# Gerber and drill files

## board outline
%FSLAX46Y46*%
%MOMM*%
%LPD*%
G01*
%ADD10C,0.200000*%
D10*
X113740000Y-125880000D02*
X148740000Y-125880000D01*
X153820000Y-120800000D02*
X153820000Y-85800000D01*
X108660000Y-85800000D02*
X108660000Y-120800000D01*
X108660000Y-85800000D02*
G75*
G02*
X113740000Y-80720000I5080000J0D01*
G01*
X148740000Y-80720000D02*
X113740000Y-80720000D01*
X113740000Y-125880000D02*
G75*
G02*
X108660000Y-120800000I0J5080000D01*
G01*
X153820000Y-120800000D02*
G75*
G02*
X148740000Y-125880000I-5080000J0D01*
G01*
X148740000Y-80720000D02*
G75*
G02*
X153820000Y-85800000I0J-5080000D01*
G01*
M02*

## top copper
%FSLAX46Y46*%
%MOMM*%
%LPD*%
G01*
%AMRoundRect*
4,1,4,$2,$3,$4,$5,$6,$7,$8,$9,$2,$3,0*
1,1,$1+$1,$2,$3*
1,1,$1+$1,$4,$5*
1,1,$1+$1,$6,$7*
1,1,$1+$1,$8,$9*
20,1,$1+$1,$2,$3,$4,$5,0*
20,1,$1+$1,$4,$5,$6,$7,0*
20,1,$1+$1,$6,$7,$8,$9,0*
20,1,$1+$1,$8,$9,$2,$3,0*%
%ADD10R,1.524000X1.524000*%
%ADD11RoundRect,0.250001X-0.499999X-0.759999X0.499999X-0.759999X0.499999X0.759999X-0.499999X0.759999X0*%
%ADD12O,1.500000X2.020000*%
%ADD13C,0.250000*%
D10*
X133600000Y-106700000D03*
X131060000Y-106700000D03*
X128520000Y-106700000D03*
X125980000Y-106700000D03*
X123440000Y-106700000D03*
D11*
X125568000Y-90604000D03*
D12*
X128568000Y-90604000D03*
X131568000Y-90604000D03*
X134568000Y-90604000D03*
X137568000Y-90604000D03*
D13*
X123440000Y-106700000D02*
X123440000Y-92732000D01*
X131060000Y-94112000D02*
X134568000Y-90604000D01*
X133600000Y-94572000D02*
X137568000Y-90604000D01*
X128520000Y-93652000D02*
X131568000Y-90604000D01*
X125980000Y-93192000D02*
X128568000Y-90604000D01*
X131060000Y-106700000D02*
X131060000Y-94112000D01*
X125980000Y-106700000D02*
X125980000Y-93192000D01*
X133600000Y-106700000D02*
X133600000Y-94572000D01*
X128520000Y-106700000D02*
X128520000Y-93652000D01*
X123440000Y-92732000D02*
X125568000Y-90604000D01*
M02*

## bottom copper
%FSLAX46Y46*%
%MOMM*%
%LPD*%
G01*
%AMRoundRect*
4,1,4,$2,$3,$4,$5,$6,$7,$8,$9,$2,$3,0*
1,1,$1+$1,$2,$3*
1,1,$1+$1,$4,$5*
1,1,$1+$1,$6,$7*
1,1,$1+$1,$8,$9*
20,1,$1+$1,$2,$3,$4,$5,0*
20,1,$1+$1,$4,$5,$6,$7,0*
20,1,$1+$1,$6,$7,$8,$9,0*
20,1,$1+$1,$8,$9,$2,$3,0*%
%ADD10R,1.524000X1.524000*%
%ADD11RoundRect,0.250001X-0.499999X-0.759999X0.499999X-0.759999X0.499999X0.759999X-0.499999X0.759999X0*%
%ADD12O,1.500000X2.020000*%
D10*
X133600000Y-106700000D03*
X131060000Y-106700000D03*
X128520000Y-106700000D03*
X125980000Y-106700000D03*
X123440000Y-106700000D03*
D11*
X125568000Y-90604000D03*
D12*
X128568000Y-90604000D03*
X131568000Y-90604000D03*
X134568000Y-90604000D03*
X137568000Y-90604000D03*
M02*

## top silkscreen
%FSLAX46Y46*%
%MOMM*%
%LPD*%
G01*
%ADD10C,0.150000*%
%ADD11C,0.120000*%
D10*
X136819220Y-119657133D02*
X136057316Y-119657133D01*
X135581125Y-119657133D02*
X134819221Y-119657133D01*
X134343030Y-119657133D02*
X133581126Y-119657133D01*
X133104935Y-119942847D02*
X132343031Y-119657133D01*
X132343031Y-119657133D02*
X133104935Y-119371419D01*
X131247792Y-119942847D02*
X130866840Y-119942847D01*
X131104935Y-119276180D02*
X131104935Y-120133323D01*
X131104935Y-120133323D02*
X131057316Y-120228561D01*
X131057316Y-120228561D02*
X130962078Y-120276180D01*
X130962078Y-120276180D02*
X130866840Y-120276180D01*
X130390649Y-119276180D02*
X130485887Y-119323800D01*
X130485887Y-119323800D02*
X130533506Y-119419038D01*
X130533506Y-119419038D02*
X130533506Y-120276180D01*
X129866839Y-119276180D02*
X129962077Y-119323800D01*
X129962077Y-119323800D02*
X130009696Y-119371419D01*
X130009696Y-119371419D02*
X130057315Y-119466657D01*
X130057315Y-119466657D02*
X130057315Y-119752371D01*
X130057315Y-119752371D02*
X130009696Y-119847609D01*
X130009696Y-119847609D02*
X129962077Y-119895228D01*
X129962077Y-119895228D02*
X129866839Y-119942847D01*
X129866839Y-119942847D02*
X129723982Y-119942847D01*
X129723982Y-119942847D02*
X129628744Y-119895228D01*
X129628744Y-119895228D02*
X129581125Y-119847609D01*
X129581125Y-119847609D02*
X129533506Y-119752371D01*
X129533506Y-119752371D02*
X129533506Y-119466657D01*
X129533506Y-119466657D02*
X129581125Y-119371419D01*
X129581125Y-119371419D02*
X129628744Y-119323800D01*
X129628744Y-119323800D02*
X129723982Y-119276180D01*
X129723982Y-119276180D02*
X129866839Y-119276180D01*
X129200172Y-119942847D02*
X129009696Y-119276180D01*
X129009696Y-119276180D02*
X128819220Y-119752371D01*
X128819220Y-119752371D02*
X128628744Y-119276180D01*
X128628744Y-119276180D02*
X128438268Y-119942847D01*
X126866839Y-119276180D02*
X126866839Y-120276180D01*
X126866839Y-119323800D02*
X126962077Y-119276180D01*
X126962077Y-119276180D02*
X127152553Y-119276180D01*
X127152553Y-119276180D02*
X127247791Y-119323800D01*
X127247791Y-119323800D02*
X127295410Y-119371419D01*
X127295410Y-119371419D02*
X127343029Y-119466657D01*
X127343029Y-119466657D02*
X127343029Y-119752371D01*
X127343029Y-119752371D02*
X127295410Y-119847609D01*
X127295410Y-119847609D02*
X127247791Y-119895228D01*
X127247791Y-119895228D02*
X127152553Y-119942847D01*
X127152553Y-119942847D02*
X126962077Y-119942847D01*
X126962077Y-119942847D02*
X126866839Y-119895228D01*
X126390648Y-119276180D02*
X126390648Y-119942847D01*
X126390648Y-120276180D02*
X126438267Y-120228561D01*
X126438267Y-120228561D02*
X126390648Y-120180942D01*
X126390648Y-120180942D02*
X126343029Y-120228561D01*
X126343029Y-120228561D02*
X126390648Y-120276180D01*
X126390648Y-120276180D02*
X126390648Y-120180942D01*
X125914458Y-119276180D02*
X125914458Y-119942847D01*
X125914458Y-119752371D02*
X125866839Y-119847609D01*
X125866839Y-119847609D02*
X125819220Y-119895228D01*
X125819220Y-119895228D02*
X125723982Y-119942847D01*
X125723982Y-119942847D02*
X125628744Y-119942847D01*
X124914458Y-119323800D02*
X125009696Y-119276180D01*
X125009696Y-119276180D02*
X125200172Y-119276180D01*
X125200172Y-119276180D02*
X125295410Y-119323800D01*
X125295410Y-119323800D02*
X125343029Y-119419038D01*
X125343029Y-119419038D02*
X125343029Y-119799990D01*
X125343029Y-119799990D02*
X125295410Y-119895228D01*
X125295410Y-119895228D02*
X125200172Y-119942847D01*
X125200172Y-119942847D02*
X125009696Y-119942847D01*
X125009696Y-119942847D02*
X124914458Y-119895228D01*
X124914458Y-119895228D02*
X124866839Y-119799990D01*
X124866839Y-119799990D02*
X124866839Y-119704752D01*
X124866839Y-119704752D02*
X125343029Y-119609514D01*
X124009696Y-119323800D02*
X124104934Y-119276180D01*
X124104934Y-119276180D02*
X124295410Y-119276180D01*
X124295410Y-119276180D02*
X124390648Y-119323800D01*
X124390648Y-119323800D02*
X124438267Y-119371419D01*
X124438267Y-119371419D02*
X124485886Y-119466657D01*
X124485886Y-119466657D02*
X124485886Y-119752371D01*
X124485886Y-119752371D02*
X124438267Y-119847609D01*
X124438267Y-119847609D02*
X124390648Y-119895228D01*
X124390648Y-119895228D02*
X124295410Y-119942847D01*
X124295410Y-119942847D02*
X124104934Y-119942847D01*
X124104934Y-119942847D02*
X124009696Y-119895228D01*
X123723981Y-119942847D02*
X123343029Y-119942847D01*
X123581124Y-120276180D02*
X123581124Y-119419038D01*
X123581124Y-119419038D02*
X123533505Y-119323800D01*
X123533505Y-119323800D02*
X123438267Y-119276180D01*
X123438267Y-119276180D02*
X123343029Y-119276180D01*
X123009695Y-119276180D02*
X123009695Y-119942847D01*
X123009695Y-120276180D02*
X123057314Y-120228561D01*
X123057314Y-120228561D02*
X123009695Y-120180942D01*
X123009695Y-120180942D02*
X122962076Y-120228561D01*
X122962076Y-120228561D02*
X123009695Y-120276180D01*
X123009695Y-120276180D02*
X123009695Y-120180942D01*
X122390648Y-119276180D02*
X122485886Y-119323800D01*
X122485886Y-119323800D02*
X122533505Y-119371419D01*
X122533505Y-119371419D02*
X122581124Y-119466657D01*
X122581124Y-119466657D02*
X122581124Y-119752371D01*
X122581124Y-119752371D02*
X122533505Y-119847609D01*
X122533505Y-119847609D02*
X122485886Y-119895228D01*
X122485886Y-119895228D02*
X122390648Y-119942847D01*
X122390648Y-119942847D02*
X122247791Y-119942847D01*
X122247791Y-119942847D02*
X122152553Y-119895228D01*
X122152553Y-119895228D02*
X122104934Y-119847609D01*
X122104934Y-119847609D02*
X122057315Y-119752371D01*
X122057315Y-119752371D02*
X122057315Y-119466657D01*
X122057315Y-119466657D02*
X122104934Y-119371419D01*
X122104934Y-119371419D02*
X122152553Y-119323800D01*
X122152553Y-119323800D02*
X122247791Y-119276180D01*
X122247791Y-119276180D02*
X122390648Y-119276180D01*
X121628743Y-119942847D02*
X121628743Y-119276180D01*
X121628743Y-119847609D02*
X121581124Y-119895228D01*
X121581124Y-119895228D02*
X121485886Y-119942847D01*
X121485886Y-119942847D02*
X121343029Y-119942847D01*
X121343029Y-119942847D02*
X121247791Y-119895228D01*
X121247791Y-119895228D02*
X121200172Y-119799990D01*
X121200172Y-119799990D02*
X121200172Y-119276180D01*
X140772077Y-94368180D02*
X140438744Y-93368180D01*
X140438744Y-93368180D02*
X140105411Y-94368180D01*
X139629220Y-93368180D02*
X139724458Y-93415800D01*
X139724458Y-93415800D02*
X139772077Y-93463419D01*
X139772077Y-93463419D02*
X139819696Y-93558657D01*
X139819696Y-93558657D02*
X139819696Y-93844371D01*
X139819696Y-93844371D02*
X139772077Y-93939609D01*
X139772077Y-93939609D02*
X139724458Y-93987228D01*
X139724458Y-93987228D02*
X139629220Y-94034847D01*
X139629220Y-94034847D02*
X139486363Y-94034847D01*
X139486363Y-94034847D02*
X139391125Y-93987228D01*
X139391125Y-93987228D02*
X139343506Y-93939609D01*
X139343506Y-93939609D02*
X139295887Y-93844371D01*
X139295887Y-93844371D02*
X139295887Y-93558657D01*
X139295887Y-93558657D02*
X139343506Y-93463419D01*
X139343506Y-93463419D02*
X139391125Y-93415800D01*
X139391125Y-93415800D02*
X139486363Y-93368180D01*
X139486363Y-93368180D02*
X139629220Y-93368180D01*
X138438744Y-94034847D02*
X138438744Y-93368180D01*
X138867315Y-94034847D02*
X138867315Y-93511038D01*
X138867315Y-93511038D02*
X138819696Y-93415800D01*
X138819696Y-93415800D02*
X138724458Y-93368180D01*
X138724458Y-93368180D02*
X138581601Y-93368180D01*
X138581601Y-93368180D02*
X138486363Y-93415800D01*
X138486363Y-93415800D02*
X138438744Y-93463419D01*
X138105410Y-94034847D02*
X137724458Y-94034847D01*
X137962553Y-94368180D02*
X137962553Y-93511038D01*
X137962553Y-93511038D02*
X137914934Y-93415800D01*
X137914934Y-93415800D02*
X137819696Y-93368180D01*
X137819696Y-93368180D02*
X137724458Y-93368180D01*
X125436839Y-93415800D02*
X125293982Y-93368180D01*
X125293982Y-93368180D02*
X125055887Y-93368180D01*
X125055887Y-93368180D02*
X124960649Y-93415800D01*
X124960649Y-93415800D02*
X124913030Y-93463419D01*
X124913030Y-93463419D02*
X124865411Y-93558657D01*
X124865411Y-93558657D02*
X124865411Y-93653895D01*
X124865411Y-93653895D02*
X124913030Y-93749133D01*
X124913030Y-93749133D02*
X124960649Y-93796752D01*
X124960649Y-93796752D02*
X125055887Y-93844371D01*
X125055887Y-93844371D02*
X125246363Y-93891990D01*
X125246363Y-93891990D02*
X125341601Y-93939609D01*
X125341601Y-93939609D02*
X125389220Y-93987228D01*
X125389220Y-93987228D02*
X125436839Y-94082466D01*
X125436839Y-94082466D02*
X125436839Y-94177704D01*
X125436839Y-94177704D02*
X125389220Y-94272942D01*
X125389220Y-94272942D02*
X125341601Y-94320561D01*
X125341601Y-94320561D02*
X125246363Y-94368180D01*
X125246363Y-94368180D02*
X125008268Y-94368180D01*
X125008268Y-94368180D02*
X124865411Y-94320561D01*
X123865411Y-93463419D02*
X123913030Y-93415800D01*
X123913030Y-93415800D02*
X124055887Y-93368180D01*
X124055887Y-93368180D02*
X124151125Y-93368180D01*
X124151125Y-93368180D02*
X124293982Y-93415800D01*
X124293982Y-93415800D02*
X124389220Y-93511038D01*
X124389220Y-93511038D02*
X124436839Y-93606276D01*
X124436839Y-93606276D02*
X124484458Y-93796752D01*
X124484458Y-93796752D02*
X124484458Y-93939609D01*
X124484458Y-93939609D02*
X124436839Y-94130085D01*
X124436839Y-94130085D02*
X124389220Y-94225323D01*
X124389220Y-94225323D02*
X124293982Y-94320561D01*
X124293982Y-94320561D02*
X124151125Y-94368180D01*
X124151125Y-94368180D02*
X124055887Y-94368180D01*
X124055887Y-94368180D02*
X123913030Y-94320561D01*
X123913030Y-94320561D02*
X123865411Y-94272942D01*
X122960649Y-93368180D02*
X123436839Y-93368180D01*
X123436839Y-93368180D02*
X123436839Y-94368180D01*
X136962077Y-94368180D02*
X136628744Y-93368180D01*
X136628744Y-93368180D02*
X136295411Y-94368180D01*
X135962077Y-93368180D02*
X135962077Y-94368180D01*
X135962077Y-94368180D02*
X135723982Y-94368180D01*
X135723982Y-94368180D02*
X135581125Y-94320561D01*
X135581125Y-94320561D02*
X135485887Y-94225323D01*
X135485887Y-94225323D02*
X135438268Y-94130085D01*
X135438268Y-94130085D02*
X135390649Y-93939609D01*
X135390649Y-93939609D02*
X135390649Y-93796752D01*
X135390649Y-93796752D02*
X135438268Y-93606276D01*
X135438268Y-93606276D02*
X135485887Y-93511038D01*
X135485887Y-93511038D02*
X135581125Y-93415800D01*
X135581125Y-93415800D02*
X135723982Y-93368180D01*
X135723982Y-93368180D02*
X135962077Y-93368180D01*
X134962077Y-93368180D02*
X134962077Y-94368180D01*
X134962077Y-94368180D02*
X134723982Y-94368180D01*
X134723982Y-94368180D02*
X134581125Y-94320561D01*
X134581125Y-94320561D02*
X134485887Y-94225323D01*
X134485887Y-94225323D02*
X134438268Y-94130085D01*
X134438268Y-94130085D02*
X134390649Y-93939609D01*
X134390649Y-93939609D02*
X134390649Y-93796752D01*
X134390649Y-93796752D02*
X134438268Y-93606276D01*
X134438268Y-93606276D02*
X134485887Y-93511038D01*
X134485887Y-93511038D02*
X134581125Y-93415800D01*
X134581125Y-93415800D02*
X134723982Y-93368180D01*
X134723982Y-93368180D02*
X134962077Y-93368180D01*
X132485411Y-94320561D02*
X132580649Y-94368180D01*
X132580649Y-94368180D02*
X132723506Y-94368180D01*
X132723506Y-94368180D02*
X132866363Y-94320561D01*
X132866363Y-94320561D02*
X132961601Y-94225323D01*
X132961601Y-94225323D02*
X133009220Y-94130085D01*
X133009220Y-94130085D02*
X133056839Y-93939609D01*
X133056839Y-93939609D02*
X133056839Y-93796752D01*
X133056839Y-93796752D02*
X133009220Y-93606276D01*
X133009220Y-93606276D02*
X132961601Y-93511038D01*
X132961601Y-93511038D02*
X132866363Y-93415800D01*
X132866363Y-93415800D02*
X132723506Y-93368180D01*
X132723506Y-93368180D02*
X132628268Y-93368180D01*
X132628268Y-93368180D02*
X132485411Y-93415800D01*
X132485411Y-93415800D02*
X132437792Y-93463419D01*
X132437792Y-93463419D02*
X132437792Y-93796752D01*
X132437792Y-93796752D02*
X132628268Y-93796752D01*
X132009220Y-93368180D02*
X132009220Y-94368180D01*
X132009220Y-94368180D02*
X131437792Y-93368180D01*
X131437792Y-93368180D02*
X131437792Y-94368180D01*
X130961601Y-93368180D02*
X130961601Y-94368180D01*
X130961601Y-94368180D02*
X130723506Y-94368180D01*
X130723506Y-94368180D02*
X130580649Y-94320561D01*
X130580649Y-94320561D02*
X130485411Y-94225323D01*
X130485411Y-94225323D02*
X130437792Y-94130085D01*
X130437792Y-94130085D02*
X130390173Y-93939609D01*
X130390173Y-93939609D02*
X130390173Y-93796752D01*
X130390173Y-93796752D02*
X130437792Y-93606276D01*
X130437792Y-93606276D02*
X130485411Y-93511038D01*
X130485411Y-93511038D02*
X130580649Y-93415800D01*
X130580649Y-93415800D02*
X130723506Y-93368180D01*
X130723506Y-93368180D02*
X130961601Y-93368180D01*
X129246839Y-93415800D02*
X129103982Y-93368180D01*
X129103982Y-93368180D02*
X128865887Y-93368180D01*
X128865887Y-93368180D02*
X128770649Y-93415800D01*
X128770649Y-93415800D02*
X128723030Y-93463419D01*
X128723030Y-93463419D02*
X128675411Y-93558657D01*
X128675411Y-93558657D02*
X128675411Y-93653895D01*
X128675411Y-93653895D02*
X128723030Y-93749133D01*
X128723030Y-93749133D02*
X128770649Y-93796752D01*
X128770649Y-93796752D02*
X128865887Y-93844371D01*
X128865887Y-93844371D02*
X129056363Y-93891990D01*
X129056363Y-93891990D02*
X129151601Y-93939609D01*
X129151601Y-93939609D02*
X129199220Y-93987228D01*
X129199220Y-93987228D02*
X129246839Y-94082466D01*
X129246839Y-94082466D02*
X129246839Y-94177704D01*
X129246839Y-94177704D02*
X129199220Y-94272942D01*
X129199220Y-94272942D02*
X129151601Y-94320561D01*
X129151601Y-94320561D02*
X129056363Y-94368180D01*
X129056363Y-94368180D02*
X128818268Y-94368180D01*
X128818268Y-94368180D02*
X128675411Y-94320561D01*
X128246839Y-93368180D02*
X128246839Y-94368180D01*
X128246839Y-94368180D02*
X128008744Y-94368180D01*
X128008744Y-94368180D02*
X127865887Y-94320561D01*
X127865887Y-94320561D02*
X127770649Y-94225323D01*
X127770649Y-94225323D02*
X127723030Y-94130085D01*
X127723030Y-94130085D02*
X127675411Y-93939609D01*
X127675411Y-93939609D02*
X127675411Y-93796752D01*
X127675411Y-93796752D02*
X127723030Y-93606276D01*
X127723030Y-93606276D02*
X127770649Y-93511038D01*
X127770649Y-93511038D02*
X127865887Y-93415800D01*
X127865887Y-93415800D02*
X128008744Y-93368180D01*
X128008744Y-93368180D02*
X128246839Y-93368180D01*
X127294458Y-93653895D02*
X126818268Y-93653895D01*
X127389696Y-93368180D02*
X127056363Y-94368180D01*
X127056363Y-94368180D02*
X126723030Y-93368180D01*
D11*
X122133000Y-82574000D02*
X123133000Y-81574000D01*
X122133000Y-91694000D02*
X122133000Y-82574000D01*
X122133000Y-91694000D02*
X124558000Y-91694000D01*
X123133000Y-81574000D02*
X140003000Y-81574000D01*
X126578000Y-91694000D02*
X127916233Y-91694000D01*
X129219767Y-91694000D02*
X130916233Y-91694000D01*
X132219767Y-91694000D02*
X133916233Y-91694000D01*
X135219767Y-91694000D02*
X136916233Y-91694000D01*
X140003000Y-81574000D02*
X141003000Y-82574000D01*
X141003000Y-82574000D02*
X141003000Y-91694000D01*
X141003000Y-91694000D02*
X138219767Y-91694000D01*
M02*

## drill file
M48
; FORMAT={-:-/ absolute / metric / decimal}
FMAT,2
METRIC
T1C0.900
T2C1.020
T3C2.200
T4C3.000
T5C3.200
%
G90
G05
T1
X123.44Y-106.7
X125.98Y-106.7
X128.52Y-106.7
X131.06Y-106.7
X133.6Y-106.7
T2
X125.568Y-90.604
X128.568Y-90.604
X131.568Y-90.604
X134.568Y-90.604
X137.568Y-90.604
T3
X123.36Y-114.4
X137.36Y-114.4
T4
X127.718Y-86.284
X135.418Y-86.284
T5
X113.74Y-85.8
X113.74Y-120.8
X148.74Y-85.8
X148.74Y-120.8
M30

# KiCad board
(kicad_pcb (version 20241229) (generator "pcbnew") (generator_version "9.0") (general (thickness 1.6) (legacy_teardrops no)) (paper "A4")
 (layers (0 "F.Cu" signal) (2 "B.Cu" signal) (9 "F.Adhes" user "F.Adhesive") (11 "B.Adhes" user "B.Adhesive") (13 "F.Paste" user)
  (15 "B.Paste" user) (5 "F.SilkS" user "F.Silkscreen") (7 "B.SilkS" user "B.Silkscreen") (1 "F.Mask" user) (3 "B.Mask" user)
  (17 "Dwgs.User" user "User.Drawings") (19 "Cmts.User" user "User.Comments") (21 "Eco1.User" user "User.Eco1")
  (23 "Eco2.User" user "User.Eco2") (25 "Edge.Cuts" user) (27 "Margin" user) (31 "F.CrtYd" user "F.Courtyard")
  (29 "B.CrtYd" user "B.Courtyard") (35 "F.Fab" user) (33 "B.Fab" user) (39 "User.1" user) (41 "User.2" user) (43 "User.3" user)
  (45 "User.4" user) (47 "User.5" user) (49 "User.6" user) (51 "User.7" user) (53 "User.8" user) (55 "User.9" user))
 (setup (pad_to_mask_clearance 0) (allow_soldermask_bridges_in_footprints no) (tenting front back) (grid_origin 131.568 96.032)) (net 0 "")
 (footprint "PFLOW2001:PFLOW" (layer "F.Cu") (at 141.22 103.5 180)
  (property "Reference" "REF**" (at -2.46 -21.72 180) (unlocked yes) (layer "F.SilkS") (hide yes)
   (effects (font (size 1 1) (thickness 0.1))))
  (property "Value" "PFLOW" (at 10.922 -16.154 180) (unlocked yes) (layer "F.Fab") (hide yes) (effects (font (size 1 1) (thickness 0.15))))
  (pad "" np_thru_hole circle (at 3.86 -10.9 180) (size 2.2 2.2) (drill 2.2) (layers "*.Cu" "*.Mask"))
  (pad "" np_thru_hole circle (at 17.86 -10.9 180) (size 2.2 2.2) (drill 2.2) (layers "*.Cu" "*.Mask"))
  (pad "1" thru_hole rect (at 7.62 -3.2 180) (size 1.524 1.524) (drill 0.9) (layers "*.Cu" "*.Mask") (remove_unused_layers no))
  (pad "2" thru_hole rect (at 10.16 -3.2 180) (size 1.524 1.524) (drill 0.9) (layers "*.Cu" "*.Mask") (remove_unused_layers no))
  (pad "3" thru_hole rect (at 12.7 -3.2 180) (size 1.524 1.524) (drill 0.9) (layers "*.Cu" "*.Mask") (remove_unused_layers no))
  (pad "4" thru_hole rect (at 15.24 -3.2 180) (size 1.524 1.524) (drill 0.9) (layers "*.Cu" "*.Mask") (remove_unused_layers no))
  (pad "5" thru_hole rect (at 17.78 -3.2 180) (size 1.524 1.524) (drill 0.9) (layers "*.Cu" "*.Mask") (remove_unused_layers no)))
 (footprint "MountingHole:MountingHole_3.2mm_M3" (layer "F.Cu") (at 113.74 120.8)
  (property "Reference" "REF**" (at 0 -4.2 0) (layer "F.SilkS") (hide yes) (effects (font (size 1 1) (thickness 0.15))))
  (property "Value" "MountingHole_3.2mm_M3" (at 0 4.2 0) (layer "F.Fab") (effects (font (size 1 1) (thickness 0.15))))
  (pad "" np_thru_hole circle (at 0 0) (size 3.2 3.2) (drill 3.2) (layers "*.Cu" "*.Mask")))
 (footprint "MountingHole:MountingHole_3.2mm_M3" (layer "F.Cu") (at 148.74 120.8)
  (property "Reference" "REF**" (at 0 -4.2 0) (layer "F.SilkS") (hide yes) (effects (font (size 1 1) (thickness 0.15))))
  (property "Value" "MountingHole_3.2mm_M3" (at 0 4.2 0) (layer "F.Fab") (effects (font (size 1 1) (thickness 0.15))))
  (pad "" np_thru_hole circle (at 0 0) (size 3.2 3.2) (drill 3.2) (layers "*.Cu" "*.Mask")))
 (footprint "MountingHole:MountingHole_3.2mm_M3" (layer "F.Cu") (at 113.74 85.8)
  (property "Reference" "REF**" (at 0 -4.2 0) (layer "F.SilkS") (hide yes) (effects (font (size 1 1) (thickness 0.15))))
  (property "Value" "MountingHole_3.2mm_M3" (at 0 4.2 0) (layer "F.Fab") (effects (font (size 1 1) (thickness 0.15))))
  (pad "" np_thru_hole circle (at 0 0) (size 3.2 3.2) (drill 3.2) (layers "*.Cu" "*.Mask")))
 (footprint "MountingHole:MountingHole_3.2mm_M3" (layer "F.Cu") (at 148.74 85.8)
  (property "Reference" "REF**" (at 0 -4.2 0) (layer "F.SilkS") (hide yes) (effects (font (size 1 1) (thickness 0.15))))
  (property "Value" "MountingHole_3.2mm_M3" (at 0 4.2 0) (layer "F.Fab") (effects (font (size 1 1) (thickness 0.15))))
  (pad "" np_thru_hole circle (at 0 0) (size 3.2 3.2) (drill 3.2) (layers "*.Cu" "*.Mask")))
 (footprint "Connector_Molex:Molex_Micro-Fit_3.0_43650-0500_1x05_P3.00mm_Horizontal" (layer "F.Cu") (at 125.568 90.604)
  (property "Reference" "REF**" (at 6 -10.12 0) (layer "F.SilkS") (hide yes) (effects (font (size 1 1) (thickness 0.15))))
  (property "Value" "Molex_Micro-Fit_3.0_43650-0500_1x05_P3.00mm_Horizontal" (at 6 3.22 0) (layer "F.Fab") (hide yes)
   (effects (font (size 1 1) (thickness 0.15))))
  (fp_line (start -3.435 -8.03) (end -2.435 -9.03) (stroke (width 0.12) (type solid)) (layer "F.SilkS"))
  (fp_line (start -3.435 1.09) (end -3.435 -8.03) (stroke (width 0.12) (type solid)) (layer "F.SilkS"))
  (fp_line (start -3.435 1.09) (end -1.01 1.09) (stroke (width 0.12) (type solid)) (layer "F.SilkS"))
  (fp_line (start -2.435 -9.03) (end 14.435 -9.03) (stroke (width 0.12) (type solid)) (layer "F.SilkS"))
  (fp_line (start 1.01 1.09) (end 2.348233 1.09) (stroke (width 0.12) (type solid)) (layer "F.SilkS"))
  (fp_line (start 3.651767 1.09) (end 5.348233 1.09) (stroke (width 0.12) (type solid)) (layer "F.SilkS"))
  (fp_line (start 6.651767 1.09) (end 8.348233 1.09) (stroke (width 0.12) (type solid)) (layer "F.SilkS"))
  (fp_line (start 9.651767 1.09) (end 11.348233 1.09) (stroke (width 0.12) (type solid)) (layer "F.SilkS"))
  (fp_line (start 14.435 -9.03) (end 15.435 -8.03) (stroke (width 0.12) (type solid)) (layer "F.SilkS"))
  (fp_line (start 15.435 -8.03) (end 15.435 1.09) (stroke (width 0.12) (type solid)) (layer "F.SilkS"))
  (fp_line (start 15.435 1.09) (end 12.651767 1.09) (stroke (width 0.12) (type solid)) (layer "F.SilkS"))
  (pad "" np_thru_hole circle (at 2.15 -4.32) (size 3 3) (drill 3) (layers "*.Cu" "*.Mask"))
  (pad "" np_thru_hole circle (at 9.85 -4.32) (size 3 3) (drill 3) (layers "*.Cu" "*.Mask"))
  (pad "1" thru_hole roundrect (at 0 0) (size 1.5 2.02) (drill 1.02) (layers "*.Cu" "*.Mask") (remove_unused_layers no)
   (roundrect_rratio 0.1666673333))
  (pad "2" thru_hole oval (at 3 0) (size 1.5 2.02) (drill 1.02) (layers "*.Cu" "*.Mask") (remove_unused_layers no))
  (pad "3" thru_hole oval (at 6 0) (size 1.5 2.02) (drill 1.02) (layers "*.Cu" "*.Mask") (remove_unused_layers no))
  (pad "4" thru_hole oval (at 9 0) (size 1.5 2.02) (drill 1.02) (layers "*.Cu" "*.Mask") (remove_unused_layers no))
  (pad "5" thru_hole oval (at 12 0) (size 1.5 2.02) (drill 1.02) (layers "*.Cu" "*.Mask") (remove_unused_layers no)))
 (gr_line (start 113.74 125.88) (end 148.74 125.88) (stroke (width 0.2) (type default)) (layer "Edge.Cuts"))
 (gr_line (start 153.82 120.8) (end 153.82 85.8) (stroke (width 0.2) (type default)) (layer "Edge.Cuts"))
 (gr_line (start 108.66 85.8) (end 108.66 120.8) (stroke (width 0.2) (type default)) (layer "Edge.Cuts"))
 (gr_arc (start 108.66 85.8) (mid 110.147898 82.207898) (end 113.74 80.72) (stroke (width 0.2) (type default)) (layer "Edge.Cuts"))
 (gr_line (start 148.74 80.72) (end 113.74 80.72) (stroke (width 0.2) (type default)) (layer "Edge.Cuts"))
 (gr_arc (start 113.74 125.88) (mid 110.147898 124.392102) (end 108.66 120.8) (stroke (width 0.2) (type default)) (layer "Edge.Cuts"))
 (gr_arc (start 153.82 120.8) (mid 152.332102 124.392102) (end 148.74 125.88) (stroke (width 0.2) (type default)) (layer "Edge.Cuts"))
 (gr_arc (start 148.74 80.72) (mid 152.332102 82.207898) (end 153.82 85.8) (stroke (width 0.2) (type default)) (layer "Edge.Cuts"))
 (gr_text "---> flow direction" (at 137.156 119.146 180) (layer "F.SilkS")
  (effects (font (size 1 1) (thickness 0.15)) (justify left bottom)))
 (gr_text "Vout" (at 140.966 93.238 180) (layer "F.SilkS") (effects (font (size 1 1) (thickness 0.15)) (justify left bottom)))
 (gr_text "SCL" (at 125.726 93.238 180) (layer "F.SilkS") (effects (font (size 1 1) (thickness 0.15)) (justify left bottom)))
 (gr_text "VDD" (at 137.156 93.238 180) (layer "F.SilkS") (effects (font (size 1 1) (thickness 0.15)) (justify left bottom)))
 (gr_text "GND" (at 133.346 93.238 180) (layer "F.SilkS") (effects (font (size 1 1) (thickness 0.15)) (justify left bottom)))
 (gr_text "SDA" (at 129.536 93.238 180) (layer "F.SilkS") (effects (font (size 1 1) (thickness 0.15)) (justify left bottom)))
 (segment (start 123.44 106.7) (end 123.44 92.732) (width 0.25) (layer "F.Cu") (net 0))
 (segment (start 131.06 94.112) (end 134.568 90.604) (width 0.25) (layer "F.Cu") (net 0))
 (segment (start 133.6 94.572) (end 137.568 90.604) (width 0.25) (layer "F.Cu") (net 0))
 (segment (start 128.52 93.652) (end 131.568 90.604) (width 0.25) (layer "F.Cu") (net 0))
 (segment (start 125.98 93.192) (end 128.568 90.604) (width 0.25) (layer "F.Cu") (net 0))
 (segment (start 131.06 106.7) (end 131.06 94.112) (width 0.25) (layer "F.Cu") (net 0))
 (segment (start 125.98 106.7) (end 125.98 93.192) (width 0.25) (layer "F.Cu") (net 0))
 (segment (start 133.6 106.7) (end 133.6 94.572) (width 0.25) (layer "F.Cu") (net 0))
 (segment (start 128.52 106.7) (end 128.52 93.652) (width 0.25) (layer "F.Cu") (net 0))
 (segment (start 123.44 92.732) (end 125.568 90.604) (width 0.25) (layer "F.Cu") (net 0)))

